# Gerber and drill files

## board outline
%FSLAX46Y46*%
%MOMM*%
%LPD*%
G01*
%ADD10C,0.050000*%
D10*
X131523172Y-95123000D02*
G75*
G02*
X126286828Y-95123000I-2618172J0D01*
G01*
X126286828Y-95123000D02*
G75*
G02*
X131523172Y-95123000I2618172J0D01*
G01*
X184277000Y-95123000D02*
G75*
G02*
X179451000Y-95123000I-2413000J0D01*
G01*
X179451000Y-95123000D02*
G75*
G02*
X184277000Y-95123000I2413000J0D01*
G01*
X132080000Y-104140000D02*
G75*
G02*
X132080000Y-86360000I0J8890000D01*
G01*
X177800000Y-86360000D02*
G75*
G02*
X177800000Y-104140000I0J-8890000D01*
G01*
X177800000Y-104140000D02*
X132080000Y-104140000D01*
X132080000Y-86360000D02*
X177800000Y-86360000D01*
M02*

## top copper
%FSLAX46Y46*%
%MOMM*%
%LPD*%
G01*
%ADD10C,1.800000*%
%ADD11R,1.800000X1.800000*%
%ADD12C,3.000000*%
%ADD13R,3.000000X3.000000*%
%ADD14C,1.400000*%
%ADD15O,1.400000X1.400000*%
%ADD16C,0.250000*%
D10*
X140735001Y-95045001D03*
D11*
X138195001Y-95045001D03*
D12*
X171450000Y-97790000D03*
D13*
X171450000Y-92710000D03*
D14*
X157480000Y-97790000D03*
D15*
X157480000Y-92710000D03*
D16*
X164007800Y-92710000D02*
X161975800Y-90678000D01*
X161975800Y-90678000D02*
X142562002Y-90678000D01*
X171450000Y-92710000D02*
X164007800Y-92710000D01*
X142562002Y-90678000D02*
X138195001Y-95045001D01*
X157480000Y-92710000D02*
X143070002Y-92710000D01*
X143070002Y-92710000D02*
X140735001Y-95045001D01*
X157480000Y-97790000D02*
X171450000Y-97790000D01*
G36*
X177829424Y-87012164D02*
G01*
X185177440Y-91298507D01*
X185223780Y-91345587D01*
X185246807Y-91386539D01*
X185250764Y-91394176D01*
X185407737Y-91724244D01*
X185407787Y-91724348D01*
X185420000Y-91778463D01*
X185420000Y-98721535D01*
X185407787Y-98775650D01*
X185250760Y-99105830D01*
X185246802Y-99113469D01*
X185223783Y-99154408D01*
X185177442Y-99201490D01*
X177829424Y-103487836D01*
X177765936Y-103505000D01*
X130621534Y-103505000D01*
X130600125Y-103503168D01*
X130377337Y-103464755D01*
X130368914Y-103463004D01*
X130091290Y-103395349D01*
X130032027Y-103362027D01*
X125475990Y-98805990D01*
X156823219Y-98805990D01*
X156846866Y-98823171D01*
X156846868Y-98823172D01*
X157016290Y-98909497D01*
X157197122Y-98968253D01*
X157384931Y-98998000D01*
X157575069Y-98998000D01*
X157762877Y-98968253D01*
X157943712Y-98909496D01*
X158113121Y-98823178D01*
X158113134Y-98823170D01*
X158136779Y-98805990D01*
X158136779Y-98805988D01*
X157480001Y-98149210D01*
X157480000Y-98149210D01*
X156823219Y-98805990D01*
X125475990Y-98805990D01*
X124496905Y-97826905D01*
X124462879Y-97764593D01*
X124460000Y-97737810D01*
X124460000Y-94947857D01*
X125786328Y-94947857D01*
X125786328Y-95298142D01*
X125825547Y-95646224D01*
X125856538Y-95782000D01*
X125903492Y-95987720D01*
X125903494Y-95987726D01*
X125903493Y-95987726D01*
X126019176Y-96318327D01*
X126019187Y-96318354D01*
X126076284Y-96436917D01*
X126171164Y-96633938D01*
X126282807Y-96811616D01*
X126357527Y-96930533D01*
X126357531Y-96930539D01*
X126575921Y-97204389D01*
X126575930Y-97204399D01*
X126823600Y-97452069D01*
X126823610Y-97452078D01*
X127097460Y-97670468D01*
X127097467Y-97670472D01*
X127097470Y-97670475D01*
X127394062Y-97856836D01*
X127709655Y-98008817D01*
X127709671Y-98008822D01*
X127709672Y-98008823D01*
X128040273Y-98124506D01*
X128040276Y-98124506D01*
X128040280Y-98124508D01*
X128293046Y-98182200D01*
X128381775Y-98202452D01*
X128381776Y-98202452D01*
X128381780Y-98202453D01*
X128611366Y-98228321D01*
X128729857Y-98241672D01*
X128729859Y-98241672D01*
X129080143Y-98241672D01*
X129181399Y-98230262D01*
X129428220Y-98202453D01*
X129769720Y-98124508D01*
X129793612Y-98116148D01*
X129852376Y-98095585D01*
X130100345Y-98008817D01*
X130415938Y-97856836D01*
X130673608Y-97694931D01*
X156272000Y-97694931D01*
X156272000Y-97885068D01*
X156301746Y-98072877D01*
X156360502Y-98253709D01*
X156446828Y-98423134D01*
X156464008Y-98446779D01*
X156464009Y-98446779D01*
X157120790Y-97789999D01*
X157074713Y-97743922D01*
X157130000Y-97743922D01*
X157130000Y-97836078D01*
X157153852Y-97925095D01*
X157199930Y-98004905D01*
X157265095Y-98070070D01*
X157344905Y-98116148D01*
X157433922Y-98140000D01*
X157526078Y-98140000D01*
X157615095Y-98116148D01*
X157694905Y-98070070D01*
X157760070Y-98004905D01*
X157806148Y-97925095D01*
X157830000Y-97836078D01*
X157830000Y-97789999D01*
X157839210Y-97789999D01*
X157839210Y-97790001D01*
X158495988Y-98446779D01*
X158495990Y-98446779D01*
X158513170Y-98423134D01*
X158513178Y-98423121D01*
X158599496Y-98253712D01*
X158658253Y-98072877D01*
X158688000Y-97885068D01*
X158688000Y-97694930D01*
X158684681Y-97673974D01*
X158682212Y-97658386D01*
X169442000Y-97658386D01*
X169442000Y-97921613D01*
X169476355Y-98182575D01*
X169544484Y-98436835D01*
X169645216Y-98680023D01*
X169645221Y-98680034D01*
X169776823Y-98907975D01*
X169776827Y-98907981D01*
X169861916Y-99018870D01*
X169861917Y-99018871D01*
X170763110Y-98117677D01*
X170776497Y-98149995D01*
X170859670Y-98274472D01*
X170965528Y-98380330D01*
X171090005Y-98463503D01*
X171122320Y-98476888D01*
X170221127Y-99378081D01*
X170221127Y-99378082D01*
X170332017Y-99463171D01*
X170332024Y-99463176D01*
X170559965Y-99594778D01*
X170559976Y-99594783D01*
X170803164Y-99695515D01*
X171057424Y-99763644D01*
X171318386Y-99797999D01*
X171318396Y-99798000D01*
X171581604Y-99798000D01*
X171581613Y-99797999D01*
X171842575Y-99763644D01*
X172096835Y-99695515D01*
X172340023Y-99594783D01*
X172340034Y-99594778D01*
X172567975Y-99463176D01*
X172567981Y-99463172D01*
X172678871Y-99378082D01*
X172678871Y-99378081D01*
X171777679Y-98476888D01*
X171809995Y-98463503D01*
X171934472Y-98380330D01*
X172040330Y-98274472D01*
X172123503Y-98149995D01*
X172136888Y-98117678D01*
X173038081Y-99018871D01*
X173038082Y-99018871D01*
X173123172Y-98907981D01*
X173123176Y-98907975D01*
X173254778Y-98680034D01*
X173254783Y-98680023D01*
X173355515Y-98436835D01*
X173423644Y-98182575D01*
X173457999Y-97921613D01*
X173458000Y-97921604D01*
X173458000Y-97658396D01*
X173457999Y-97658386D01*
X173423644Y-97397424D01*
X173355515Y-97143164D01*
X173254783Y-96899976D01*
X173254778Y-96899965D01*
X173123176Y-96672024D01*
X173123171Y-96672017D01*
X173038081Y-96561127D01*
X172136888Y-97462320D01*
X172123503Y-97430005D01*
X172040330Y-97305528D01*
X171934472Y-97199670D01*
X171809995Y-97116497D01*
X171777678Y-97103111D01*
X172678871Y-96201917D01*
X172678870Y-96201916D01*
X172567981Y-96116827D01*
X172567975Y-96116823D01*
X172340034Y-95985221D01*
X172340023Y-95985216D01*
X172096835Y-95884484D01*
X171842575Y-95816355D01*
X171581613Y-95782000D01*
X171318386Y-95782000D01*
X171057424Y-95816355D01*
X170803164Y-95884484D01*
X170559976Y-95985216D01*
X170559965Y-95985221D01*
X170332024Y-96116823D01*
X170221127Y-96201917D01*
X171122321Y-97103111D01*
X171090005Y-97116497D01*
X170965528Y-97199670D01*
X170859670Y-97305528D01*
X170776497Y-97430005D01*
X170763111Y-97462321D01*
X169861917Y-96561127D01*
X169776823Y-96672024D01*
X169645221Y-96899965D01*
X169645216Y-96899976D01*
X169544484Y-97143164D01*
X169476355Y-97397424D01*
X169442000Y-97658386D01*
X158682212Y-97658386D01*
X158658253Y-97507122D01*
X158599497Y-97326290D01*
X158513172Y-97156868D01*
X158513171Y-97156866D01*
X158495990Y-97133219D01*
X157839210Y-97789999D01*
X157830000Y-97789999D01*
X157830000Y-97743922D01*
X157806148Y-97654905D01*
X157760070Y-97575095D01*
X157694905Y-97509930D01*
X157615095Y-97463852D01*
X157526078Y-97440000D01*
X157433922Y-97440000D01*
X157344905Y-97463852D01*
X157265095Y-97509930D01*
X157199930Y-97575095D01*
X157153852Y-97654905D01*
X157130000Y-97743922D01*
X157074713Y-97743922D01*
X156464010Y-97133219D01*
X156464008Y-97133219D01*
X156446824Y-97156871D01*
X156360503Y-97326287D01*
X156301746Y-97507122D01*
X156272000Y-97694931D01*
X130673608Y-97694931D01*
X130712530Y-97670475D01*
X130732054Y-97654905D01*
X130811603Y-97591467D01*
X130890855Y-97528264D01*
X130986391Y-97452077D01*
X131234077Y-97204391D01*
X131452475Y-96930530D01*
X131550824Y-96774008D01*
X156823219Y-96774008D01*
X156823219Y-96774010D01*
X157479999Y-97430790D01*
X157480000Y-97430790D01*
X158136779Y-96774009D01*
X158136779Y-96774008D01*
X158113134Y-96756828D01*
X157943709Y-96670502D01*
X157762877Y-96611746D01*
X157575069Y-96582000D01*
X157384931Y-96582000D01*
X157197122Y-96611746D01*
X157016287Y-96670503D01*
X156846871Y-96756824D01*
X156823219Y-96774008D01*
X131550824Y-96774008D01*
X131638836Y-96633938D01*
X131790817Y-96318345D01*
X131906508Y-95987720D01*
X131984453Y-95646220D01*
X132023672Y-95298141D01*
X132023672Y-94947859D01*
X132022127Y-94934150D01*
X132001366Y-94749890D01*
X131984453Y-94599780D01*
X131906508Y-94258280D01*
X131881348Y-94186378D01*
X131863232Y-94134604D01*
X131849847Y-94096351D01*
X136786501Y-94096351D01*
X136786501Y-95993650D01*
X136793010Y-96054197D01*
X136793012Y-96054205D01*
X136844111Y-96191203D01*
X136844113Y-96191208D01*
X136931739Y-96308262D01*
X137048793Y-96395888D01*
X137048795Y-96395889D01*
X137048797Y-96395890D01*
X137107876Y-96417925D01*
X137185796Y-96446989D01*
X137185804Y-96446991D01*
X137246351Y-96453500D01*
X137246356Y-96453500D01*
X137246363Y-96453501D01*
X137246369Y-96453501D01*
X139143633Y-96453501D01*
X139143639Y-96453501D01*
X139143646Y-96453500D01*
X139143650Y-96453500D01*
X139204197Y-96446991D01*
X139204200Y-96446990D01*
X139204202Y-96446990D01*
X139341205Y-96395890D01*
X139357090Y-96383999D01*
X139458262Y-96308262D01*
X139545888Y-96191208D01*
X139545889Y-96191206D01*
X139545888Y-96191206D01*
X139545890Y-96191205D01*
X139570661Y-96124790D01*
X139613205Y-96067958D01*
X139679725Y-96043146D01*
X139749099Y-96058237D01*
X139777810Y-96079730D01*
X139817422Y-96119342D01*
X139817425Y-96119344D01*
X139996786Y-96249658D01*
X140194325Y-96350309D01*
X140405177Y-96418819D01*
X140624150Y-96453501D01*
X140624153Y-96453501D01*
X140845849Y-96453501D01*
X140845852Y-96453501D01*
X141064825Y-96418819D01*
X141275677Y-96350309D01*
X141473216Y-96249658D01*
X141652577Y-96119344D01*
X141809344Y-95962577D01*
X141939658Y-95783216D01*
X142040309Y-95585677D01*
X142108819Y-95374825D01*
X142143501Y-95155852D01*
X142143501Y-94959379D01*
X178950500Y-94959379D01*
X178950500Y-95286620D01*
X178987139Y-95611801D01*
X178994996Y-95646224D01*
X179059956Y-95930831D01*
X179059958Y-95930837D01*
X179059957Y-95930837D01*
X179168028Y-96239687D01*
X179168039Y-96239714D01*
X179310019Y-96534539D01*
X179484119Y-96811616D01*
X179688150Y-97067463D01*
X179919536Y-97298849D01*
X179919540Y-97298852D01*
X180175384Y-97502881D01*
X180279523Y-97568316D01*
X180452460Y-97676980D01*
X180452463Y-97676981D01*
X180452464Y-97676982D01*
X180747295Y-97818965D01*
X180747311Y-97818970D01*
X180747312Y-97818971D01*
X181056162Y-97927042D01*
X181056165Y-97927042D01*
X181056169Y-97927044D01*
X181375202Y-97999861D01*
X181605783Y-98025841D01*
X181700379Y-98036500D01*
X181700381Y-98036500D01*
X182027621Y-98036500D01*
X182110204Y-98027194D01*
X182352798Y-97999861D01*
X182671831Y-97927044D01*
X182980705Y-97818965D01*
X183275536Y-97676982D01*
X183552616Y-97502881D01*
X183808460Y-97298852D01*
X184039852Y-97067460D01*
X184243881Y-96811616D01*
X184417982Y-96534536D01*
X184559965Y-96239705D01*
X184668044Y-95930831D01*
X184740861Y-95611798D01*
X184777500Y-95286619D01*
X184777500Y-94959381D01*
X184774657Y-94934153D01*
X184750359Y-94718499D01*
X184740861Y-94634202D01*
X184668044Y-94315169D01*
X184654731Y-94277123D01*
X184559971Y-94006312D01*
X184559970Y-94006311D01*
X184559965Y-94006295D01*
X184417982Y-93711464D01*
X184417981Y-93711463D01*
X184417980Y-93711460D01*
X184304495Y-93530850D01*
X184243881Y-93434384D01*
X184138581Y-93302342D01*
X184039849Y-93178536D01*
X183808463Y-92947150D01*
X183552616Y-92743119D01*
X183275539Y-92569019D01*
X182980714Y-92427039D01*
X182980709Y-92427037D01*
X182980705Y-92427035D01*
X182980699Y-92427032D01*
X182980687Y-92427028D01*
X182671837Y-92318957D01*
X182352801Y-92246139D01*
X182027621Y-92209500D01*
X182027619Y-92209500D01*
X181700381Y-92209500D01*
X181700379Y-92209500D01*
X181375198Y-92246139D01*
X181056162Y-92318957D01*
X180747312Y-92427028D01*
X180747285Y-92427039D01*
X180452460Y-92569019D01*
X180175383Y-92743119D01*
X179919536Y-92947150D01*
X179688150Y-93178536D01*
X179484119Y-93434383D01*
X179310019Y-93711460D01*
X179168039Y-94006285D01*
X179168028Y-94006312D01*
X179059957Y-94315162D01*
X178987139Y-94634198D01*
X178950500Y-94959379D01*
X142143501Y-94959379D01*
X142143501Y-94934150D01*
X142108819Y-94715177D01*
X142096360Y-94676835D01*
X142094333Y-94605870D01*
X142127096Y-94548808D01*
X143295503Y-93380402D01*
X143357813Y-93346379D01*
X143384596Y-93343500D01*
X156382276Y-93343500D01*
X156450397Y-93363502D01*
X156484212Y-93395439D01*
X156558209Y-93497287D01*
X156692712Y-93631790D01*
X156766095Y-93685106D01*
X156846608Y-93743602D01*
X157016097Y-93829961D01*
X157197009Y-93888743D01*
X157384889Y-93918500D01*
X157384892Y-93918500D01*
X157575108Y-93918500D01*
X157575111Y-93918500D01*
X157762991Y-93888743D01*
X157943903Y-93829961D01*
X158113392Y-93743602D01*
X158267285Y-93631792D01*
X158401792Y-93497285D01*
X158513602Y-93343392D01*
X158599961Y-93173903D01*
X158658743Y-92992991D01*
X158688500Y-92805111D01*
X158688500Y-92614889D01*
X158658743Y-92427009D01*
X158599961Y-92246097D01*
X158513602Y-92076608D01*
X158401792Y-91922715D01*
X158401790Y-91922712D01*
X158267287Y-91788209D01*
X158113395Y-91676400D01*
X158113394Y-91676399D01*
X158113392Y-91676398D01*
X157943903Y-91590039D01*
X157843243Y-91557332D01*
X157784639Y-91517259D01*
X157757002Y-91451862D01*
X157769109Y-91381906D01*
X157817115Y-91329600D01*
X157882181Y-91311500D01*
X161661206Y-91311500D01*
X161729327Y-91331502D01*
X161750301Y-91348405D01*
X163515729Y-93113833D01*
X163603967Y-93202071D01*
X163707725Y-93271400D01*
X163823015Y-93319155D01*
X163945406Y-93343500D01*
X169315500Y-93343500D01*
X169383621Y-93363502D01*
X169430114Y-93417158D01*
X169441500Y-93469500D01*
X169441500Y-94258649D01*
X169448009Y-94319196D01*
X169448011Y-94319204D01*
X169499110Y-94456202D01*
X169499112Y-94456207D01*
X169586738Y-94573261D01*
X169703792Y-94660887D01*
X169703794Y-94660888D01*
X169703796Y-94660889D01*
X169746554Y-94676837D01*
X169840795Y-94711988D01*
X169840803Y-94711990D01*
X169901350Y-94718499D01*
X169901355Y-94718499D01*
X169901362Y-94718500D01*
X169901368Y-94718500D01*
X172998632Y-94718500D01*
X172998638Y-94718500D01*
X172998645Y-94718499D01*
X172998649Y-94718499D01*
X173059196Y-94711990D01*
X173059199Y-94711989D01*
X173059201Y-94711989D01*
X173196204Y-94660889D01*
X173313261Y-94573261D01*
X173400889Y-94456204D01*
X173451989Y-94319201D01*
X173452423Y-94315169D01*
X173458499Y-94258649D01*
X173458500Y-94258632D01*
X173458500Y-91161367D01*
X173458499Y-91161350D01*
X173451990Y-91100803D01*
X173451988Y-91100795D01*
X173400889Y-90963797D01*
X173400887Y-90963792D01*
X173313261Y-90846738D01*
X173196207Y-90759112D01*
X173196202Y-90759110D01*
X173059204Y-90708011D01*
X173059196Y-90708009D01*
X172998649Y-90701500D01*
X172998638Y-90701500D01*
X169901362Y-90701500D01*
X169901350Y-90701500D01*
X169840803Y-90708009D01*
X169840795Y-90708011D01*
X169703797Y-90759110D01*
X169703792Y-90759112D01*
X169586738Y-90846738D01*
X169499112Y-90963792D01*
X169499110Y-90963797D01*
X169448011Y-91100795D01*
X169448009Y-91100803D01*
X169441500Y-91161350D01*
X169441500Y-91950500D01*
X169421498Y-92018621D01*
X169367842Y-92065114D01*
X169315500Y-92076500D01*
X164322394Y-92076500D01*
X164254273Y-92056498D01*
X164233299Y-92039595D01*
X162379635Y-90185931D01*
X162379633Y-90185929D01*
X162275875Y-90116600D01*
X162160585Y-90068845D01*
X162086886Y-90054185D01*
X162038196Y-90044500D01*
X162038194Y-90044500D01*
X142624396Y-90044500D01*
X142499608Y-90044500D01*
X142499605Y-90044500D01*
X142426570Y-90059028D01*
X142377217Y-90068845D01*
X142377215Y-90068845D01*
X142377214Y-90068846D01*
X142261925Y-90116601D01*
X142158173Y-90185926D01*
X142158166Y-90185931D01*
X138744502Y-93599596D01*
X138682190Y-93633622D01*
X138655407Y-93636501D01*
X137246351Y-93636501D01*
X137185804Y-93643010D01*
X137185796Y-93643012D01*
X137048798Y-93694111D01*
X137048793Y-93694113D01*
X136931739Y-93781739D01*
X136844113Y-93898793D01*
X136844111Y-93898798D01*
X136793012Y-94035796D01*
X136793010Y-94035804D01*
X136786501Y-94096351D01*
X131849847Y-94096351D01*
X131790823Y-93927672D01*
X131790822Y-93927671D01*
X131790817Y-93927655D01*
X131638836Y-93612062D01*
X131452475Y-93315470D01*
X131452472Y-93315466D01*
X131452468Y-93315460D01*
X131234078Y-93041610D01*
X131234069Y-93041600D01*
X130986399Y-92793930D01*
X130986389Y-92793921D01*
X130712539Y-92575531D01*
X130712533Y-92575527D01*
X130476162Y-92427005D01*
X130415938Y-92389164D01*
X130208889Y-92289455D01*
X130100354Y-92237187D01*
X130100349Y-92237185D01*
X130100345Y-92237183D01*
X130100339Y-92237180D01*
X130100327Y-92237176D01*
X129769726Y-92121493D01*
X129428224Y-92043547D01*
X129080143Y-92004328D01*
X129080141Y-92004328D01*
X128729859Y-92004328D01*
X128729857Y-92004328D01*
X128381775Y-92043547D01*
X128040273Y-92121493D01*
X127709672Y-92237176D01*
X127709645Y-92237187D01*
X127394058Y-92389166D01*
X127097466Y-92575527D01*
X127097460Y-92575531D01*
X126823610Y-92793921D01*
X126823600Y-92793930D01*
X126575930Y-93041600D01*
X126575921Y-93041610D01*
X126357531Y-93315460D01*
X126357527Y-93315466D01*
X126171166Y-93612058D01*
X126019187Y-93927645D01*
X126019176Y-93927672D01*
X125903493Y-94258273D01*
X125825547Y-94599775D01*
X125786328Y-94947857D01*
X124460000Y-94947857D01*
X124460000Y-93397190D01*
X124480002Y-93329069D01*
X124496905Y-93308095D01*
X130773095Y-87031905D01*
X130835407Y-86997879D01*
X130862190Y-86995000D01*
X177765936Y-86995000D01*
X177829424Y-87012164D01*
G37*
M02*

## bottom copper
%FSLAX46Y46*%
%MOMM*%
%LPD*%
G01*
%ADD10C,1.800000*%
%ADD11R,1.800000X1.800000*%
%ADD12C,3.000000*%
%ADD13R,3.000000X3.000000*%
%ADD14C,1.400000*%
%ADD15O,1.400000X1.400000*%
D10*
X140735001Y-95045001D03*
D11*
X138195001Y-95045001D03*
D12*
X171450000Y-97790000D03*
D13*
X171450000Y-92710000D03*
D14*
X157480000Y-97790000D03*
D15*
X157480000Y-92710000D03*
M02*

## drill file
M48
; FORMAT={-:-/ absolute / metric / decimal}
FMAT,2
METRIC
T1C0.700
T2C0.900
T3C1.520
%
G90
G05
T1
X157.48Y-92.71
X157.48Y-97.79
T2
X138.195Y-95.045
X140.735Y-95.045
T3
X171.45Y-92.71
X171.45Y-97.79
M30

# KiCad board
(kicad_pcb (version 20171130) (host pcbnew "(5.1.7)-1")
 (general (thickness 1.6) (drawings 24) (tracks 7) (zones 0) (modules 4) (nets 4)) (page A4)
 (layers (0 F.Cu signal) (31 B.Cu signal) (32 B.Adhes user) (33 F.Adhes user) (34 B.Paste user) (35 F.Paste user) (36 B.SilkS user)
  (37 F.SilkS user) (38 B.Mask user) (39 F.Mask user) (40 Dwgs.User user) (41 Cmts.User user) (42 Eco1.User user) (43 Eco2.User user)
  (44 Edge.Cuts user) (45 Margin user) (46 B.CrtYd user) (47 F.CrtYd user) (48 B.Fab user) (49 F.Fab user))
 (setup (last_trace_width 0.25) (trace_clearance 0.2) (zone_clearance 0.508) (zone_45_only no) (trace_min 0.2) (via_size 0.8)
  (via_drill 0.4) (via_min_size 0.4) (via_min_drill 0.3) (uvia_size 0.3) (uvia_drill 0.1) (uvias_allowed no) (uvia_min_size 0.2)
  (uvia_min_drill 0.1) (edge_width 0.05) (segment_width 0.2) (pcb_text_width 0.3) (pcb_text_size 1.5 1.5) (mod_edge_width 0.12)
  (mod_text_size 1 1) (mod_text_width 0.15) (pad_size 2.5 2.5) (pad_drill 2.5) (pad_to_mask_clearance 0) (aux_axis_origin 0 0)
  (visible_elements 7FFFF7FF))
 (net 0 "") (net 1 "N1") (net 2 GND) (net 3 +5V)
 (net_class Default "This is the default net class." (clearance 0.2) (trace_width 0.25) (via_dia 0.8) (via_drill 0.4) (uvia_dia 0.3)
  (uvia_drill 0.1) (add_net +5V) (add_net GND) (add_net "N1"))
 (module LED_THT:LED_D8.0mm (layer F.Cu) (at 138.195001 95.045001)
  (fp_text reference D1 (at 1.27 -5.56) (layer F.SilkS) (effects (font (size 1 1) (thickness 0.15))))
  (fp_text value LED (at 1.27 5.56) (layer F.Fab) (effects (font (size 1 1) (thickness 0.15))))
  (pad 2 thru_hole circle (at 2.54 0) (size 1.8 1.8) (drill 0.9) (layers *.Cu *.Mask) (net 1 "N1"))
  (pad 1 thru_hole rect (at 0 0) (size 1.8 1.8) (drill 0.9) (layers *.Cu *.Mask) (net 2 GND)))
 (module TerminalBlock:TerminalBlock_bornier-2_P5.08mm (layer F.Cu) (at 171.45 92.71 270)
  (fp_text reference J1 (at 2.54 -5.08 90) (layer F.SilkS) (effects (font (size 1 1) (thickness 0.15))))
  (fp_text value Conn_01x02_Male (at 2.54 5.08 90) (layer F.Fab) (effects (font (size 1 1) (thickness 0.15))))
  (pad 2 thru_hole circle (at 5.08 0 270) (size 3 3) (drill 1.52) (layers *.Cu *.Mask) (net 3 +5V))
  (pad 1 thru_hole rect (at 0 0 270) (size 3 3) (drill 1.52) (layers *.Cu *.Mask) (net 2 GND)))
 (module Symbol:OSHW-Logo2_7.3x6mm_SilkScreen (layer B.Cu) (at 163.83 95.25 270)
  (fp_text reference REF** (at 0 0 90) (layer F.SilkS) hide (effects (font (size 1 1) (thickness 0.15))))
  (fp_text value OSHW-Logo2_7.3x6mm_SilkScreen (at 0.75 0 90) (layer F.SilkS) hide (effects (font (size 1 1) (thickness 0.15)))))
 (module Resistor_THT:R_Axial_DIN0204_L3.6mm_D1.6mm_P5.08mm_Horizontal (layer F.Cu) (at 157.48 97.79 90)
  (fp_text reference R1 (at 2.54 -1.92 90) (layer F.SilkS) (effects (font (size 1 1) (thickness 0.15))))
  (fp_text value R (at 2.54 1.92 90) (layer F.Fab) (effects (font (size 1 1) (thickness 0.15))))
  (pad 1 thru_hole circle (at 0 0 90) (size 1.4 1.4) (drill 0.7) (layers *.Cu *.Mask) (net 3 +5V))
  (pad 2 thru_hole oval (at 5.08 0 90) (size 1.4 1.4) (drill 0.7) (layers *.Cu *.Mask) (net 1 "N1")))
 (gr_circle (center 128.905 95.123) (end 127.254 93.091) (layer Edge.Cuts) (width 0.05))
 (gr_circle (center 181.864 95.123) (end 181.864 92.71) (layer Edge.Cuts) (width 0.05))
 (gr_arc (start 132.08 95.25) (end 132.08 86.36) (angle -180) (layer Edge.Cuts) (width 0.05))
 (gr_arc (start 177.8 95.25) (end 177.8 104.14) (angle -180) (layer Edge.Cuts) (width 0.05))
 (gr_line (start 177.8 104.14) (end 132.08 104.14) (layer Edge.Cuts) (width 0.05))
 (gr_line (start 132.08 86.36) (end 177.8 86.36) (layer Edge.Cuts) (width 0.05))
 (segment (start 164.0078 92.71) (end 161.9758 90.678) (width 0.25) (layer F.Cu) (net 2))
 (segment (start 161.9758 90.678) (end 142.562002 90.678) (width 0.25) (layer F.Cu) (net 2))
 (segment (start 171.45 92.71) (end 164.0078 92.71) (width 0.25) (layer F.Cu) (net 2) (status 400010))
 (segment (start 142.562002 90.678) (end 138.195001 95.045001) (width 0.25) (layer F.Cu) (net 2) (status 800020))
 (segment (start 157.48 92.71) (end 143.070002 92.71) (width 0.25) (layer F.Cu) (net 1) (status 10))
 (segment (start 143.070002 92.71) (end 140.735001 95.045001) (width 0.25) (layer F.Cu) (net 1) (status 20))
 (segment (start 157.48 97.79) (end 171.45 97.79) (width 0.25) (layer F.Cu) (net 3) (status C00030))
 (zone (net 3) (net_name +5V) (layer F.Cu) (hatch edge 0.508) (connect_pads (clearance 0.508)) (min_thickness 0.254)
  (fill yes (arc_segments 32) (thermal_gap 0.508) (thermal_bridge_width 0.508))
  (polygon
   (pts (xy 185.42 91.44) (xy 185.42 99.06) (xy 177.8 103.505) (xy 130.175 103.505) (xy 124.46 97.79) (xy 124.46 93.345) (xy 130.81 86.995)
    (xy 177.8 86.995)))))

